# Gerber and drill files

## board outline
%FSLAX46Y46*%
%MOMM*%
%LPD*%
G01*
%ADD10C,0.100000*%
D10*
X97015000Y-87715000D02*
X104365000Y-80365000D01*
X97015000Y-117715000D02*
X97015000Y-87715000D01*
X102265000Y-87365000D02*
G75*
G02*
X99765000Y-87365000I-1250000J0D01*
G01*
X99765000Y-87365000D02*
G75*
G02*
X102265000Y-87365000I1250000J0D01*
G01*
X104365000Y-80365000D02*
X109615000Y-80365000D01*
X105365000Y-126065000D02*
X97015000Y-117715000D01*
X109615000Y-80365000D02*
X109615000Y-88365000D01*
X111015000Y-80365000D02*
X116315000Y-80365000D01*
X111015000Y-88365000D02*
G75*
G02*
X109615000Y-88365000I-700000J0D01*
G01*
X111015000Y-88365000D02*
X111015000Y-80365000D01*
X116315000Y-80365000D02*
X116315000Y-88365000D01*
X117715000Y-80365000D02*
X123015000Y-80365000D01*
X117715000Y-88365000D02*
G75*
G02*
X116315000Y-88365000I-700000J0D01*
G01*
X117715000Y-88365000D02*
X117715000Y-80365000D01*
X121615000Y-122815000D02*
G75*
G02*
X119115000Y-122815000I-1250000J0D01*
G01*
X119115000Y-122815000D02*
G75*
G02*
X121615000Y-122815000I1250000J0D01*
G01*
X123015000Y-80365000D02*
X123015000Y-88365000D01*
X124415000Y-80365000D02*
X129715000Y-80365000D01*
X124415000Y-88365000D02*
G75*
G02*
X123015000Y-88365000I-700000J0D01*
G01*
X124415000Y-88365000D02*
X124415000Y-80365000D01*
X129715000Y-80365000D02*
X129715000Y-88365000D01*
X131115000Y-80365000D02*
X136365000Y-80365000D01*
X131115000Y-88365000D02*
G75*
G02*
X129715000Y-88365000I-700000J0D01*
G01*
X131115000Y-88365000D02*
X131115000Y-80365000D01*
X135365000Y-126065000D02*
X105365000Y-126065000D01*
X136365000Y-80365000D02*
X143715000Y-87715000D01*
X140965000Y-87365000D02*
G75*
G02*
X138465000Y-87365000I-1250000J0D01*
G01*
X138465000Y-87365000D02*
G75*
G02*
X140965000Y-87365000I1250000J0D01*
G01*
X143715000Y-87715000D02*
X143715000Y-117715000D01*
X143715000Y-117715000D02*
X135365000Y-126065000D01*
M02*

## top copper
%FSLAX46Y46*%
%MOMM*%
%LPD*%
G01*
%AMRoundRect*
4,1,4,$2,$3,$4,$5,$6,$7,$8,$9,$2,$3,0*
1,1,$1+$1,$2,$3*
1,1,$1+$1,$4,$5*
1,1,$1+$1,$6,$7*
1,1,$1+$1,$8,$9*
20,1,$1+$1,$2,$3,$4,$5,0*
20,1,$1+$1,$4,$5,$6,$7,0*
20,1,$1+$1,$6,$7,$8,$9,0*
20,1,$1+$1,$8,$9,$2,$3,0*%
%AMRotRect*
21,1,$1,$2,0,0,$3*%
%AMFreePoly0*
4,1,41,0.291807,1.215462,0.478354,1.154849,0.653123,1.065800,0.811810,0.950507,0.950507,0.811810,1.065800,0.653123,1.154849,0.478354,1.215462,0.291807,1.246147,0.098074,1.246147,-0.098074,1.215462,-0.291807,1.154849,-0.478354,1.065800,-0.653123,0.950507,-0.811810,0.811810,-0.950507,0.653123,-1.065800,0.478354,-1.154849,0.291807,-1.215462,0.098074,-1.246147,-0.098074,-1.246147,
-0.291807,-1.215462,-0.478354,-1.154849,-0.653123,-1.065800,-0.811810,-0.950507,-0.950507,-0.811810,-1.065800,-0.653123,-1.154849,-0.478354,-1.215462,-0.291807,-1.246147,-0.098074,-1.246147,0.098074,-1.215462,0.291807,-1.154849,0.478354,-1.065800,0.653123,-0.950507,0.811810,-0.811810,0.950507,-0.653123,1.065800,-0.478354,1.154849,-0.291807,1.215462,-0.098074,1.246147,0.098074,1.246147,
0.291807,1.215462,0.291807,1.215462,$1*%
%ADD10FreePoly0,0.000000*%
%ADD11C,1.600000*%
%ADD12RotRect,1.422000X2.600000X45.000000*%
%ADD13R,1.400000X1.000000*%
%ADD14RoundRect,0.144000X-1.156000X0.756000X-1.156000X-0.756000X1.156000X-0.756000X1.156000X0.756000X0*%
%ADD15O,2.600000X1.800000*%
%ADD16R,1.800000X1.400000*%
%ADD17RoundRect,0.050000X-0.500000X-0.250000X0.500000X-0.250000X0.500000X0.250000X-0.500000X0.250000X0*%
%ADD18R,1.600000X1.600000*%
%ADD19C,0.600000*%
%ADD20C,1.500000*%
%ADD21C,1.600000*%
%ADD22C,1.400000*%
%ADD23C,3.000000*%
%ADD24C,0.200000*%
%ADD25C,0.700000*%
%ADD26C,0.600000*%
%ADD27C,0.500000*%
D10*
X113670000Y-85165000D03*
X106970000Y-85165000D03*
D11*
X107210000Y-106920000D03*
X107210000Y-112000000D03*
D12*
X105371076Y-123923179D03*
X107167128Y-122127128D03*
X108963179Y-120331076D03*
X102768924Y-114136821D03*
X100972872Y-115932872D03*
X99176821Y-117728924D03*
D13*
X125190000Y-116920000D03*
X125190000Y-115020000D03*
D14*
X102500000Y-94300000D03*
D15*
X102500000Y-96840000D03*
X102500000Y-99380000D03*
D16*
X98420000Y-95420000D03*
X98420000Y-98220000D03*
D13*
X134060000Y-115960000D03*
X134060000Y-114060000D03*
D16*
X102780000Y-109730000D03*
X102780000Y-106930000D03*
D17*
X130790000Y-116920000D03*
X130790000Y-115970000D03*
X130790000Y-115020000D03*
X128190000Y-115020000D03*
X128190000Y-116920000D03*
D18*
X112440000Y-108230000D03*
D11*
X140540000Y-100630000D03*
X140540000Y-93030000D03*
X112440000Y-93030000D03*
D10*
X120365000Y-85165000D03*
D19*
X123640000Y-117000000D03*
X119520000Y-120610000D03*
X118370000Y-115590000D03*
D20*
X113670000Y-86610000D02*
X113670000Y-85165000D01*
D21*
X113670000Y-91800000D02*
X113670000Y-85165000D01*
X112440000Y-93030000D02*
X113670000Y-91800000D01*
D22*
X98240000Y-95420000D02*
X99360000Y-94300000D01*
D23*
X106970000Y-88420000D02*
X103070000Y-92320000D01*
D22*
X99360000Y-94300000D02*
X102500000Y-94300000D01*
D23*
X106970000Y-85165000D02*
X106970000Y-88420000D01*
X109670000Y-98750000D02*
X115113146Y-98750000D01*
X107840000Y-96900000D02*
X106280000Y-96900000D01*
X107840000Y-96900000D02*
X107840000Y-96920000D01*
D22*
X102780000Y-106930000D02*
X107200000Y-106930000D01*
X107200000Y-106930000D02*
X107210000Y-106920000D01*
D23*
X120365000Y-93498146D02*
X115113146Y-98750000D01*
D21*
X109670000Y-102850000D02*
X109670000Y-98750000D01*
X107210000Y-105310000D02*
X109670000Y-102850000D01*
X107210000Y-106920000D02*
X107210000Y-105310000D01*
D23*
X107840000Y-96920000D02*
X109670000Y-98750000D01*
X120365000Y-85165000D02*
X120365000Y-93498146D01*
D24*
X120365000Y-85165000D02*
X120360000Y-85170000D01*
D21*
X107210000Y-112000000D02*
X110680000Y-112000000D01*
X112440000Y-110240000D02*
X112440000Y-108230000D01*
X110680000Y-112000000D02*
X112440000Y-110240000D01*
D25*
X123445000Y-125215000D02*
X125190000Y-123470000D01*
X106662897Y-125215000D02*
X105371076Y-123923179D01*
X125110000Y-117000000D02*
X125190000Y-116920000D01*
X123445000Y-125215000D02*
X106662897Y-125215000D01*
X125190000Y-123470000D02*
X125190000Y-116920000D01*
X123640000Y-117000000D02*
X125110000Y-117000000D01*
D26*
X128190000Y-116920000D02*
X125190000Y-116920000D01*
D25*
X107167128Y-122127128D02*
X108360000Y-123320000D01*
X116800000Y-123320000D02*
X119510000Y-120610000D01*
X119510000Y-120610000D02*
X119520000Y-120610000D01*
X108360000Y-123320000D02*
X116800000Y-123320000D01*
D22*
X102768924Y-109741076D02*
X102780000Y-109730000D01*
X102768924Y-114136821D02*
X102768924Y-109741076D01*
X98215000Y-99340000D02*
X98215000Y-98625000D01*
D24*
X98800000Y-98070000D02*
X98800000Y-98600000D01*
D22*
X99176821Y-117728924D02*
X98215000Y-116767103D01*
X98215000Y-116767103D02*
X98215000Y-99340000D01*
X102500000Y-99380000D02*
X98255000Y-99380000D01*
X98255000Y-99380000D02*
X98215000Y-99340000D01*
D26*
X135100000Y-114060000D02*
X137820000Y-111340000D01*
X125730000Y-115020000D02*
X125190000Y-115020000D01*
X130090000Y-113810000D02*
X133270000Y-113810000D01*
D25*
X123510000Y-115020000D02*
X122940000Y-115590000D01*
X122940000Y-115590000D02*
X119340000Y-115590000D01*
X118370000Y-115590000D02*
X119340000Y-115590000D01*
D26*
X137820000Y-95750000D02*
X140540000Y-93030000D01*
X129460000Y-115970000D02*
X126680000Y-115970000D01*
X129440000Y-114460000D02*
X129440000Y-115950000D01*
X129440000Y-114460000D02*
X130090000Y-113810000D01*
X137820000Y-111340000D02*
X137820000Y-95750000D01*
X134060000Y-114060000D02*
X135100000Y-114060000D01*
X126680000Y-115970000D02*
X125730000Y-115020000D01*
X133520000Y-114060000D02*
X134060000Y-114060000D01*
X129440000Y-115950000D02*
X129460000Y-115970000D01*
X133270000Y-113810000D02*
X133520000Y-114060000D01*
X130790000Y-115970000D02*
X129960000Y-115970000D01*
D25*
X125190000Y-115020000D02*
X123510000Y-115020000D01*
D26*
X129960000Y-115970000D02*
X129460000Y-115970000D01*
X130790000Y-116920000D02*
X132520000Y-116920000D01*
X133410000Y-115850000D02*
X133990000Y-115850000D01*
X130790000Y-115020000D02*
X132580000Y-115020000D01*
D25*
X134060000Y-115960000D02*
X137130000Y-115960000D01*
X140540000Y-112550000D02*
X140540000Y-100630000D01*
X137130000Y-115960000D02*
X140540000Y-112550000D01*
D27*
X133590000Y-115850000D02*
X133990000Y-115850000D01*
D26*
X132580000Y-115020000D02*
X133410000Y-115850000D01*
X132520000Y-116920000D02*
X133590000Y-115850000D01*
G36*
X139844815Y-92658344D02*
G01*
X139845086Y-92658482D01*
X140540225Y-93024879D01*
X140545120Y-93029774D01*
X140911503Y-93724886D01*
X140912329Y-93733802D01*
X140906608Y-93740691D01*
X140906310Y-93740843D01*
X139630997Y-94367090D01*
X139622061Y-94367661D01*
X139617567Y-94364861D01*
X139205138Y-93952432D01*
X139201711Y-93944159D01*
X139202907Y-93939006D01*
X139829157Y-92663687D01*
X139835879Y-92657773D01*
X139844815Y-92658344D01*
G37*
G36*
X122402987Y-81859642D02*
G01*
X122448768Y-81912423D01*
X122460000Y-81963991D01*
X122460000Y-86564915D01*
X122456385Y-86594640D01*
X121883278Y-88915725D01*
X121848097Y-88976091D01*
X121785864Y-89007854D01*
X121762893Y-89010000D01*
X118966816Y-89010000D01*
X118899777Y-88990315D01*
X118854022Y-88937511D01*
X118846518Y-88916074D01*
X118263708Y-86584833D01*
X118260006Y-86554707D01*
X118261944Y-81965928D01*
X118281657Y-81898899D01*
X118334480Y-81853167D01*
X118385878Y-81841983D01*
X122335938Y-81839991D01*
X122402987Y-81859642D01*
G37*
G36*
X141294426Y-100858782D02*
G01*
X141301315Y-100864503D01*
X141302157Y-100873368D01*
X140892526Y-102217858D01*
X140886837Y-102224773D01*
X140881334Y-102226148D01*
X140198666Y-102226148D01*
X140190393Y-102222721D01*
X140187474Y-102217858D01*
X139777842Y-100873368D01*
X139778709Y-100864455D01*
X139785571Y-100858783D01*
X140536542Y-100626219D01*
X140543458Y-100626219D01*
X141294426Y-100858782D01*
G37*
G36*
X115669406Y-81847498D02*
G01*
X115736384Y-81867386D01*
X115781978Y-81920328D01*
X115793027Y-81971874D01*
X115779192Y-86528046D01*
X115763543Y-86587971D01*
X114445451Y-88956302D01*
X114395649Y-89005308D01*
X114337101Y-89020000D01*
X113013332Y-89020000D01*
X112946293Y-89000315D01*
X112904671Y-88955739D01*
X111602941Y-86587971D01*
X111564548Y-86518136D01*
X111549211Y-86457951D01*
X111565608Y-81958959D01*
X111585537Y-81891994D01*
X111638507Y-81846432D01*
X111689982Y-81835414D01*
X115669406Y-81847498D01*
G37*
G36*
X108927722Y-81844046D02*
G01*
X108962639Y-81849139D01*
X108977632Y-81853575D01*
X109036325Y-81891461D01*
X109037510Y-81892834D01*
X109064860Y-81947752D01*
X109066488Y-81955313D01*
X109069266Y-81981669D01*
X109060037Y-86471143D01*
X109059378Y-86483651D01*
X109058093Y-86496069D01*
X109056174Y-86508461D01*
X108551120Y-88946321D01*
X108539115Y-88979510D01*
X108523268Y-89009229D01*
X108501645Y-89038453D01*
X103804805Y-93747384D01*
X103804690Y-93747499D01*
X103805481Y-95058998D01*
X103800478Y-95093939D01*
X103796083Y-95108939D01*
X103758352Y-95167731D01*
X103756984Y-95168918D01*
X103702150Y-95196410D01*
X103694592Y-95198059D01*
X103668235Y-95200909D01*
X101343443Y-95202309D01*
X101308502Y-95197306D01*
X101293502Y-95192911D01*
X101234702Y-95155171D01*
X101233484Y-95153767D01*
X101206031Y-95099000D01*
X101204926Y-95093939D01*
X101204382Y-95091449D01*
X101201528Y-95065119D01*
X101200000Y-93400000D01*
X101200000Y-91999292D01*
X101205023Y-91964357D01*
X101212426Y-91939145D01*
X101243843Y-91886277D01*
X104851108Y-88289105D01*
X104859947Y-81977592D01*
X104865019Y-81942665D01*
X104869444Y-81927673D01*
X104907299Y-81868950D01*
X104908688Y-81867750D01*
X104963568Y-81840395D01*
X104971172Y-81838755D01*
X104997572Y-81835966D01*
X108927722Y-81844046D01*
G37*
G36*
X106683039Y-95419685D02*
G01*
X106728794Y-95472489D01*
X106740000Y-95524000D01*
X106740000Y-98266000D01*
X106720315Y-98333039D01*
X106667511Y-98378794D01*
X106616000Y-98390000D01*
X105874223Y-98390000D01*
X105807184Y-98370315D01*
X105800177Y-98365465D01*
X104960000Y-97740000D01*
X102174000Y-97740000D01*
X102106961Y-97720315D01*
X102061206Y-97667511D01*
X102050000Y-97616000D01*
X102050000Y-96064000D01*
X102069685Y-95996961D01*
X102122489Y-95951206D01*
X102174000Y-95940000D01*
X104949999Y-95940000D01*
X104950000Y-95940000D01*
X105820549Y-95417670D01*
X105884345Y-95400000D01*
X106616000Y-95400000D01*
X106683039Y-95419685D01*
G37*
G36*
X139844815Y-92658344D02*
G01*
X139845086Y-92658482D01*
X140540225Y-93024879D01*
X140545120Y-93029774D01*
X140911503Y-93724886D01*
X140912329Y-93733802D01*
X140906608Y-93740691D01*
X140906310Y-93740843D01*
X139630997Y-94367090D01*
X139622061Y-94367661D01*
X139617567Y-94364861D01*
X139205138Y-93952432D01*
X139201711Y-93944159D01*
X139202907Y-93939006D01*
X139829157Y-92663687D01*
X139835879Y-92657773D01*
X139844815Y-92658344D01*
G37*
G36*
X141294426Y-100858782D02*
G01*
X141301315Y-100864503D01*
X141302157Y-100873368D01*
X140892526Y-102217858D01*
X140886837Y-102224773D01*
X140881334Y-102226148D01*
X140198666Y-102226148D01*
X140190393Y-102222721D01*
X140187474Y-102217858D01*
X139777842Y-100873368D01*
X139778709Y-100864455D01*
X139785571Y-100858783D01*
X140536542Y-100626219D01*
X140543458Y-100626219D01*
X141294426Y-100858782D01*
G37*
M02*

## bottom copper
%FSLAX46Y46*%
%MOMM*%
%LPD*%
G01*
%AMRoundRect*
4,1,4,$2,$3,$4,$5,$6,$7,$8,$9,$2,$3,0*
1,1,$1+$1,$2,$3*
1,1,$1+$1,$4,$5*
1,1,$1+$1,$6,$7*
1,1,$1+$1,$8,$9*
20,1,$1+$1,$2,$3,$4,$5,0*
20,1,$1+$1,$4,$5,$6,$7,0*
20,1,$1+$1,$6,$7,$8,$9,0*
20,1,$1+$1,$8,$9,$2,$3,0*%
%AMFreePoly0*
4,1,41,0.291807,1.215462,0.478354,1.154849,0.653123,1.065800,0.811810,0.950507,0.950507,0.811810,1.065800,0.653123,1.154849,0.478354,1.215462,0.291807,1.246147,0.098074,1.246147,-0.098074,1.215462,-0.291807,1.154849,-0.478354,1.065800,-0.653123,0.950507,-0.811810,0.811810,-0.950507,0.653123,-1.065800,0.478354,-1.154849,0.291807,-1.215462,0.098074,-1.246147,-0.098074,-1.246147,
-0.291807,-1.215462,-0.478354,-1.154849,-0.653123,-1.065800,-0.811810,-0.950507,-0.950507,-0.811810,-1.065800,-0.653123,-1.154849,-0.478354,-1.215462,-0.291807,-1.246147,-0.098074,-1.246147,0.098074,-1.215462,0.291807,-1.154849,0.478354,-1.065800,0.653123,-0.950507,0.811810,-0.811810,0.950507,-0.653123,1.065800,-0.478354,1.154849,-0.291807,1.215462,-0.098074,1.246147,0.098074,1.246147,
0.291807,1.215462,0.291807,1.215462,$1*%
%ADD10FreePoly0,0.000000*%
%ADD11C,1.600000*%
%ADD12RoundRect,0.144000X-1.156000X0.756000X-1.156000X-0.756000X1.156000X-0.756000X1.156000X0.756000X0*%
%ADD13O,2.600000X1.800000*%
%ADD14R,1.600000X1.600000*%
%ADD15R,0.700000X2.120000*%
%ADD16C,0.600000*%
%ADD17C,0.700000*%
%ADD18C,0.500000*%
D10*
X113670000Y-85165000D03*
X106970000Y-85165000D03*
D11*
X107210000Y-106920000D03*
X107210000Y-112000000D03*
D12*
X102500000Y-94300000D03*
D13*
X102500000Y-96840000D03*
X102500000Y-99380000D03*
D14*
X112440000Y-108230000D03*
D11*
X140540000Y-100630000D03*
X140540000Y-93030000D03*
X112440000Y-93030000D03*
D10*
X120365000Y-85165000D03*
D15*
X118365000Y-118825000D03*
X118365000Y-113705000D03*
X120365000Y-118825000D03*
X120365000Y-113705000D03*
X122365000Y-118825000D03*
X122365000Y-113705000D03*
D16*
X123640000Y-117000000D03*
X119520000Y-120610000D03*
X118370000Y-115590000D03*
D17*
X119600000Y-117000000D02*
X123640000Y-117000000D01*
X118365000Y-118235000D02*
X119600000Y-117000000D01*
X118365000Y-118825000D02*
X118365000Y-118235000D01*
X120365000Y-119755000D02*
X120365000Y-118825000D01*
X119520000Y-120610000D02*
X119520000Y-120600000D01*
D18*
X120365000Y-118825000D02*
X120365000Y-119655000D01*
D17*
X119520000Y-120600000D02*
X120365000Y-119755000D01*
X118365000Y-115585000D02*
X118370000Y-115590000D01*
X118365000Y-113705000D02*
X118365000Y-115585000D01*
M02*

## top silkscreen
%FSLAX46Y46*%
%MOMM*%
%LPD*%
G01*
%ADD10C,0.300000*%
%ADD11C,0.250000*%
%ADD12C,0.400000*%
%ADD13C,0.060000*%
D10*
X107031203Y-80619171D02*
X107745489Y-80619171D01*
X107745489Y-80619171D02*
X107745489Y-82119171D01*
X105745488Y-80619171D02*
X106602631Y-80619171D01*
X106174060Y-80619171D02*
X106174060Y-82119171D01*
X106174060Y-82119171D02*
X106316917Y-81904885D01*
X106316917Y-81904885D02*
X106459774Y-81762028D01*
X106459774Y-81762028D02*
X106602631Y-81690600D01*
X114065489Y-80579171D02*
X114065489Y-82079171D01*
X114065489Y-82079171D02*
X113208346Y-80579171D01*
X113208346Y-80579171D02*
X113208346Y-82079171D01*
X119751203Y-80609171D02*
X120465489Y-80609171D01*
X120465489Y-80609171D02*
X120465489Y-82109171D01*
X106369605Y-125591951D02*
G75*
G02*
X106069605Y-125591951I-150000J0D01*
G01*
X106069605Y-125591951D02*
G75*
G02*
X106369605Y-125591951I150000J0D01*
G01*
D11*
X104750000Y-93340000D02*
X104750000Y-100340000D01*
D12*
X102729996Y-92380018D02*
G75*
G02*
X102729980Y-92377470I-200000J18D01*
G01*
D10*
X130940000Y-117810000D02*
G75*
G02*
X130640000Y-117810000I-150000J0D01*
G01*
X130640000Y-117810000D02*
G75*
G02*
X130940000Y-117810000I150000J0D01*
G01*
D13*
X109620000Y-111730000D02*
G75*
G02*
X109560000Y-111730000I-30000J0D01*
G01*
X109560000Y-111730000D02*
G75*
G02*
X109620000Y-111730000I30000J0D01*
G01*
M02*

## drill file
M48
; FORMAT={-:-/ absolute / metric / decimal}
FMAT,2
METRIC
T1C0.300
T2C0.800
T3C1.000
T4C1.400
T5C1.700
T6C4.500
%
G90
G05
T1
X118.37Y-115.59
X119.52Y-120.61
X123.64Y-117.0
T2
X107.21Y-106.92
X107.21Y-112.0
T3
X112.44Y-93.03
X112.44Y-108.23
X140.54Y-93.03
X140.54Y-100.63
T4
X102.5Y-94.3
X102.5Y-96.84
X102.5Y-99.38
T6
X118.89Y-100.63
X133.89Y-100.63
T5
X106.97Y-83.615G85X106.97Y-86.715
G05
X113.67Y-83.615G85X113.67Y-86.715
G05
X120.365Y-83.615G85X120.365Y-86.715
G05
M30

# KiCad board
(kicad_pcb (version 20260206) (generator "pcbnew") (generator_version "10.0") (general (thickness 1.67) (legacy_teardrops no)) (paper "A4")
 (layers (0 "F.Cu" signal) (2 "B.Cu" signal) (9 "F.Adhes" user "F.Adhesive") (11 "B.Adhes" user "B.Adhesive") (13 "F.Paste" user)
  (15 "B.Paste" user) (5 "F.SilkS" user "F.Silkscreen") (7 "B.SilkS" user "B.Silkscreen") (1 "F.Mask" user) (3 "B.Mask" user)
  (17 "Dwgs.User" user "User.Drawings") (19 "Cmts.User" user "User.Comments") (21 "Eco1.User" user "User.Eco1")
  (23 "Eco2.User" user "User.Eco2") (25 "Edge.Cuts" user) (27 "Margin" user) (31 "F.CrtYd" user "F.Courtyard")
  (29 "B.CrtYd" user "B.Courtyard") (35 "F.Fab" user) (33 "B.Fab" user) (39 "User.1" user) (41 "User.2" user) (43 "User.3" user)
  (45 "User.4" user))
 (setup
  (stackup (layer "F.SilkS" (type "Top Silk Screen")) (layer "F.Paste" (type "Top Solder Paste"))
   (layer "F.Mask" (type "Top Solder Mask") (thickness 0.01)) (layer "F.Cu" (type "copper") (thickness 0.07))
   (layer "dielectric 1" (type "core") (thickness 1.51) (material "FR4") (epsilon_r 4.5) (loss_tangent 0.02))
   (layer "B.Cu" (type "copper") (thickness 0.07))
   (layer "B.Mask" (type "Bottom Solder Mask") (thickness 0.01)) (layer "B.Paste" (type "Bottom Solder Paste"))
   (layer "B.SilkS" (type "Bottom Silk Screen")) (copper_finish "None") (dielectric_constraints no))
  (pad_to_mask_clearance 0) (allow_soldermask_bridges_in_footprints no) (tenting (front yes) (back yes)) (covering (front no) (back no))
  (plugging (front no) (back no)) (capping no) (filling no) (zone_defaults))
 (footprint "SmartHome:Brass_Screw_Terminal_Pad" (layer "F.Cu") (at 113.67 85.165)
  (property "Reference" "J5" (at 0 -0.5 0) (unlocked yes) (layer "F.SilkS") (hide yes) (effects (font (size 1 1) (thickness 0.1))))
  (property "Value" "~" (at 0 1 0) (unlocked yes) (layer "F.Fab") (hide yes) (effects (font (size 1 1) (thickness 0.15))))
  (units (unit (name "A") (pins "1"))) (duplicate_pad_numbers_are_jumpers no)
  (pad "1" thru_hole custom (at 0 0) (size 2.5 2.5) (drill oval 1.7 4.8) (layers "*.Cu" "*.Mask") (remove_unused_layers no) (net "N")
   (options (clearance outline) (anchor circle)) (primitives)))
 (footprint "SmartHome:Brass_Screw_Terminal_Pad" (layer "F.Cu") (at 106.97 85.165)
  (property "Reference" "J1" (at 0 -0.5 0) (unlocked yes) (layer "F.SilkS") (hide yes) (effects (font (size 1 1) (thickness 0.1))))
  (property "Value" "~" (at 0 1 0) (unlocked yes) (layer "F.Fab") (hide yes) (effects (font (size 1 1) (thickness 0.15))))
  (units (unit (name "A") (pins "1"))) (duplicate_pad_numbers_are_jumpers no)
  (pad "1" thru_hole custom (at 0 0) (size 2.5 2.5) (drill oval 1.7 4.8) (layers "*.Cu" "*.Mask") (remove_unused_layers no) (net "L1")
   (options (clearance outline) (anchor circle)) (primitives)))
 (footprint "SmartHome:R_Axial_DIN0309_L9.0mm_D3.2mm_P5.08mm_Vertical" (layer "F.Cu") (at 107.21 106.92 -90)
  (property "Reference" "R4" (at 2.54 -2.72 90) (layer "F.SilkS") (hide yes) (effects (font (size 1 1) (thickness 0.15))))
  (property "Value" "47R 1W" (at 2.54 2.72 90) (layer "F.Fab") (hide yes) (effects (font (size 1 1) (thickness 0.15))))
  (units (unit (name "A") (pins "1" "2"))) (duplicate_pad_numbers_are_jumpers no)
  (pad "1" thru_hole circle (at 0 0 270) (size 1.6 1.6) (drill 0.8) (layers "*.Cu" "*.Mask") (remove_unused_layers no) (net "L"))
  (pad "2" thru_hole circle (at 5.08 0 270) (size 1.6 1.6) (drill 0.8) (layers "*.Cu" "*.Mask") (remove_unused_layers no)
   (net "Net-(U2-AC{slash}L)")))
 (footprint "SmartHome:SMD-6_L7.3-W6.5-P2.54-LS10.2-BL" (layer "F.Cu") (at 104.07 119.03 45)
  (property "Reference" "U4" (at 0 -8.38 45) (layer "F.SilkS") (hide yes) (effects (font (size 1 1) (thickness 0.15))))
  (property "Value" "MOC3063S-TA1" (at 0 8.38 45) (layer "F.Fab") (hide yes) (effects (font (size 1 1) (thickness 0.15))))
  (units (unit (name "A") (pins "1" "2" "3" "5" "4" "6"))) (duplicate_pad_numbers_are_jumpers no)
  (fp_circle (center -3.12 6.16) (end -2.97 6.16) (stroke (width 0.3) (type solid)) (fill no) (layer "F.SilkS"))
  (pad "1" smd rect (at -2.54 4.38 45) (size 1.422 2.6) (layers "F.Cu" "F.Mask" "F.Paste") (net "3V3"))
  (pad "2" smd rect (at 0 4.38 45) (size 1.422 2.6) (layers "F.Cu" "F.Mask" "F.Paste") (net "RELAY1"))
  (pad "3" smd rect (at 2.54 4.38 45) (size 1.422 2.6) (layers "F.Cu" "F.Mask" "F.Paste") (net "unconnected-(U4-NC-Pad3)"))
  (pad "4" smd rect (at 2.54 -4.38 45) (size 1.422 2.6) (layers "F.Cu" "F.Mask" "F.Paste") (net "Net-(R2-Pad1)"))
  (pad "5" smd rect (at 0 -4.38 45) (size 1.422 2.6) (layers "F.Cu" "F.Mask" "F.Paste") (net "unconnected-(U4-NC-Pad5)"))
  (pad "6" smd rect (at -2.54 -4.38 45) (size 1.422 2.6) (layers "F.Cu" "F.Mask" "F.Paste") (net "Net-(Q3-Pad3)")))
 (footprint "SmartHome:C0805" (layer "F.Cu") (at 125.19 115.97 90)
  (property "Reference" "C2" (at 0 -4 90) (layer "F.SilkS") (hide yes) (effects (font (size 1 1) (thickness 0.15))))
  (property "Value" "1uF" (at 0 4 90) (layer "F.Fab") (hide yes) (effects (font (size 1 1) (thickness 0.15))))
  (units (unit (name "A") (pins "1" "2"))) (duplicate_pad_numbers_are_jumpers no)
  (pad "1" smd rect (at -0.95 0 90) (size 1 1.4) (layers "F.Cu" "F.Mask" "F.Paste") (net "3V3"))
  (pad "2" smd rect (at 0.95 0 90) (size 1 1.4) (layers "F.Cu" "F.Mask" "F.Paste") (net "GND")))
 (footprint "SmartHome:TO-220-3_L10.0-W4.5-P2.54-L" (layer "F.Cu") (at 102.5 96.84 -90)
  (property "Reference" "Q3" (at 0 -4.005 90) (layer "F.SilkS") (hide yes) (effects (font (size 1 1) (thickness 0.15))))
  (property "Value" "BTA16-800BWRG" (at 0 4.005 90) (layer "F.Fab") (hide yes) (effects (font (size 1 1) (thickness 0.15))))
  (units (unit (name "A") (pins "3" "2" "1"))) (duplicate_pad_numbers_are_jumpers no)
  (fp_line (start -3.5 -2.25) (end 3.5 -2.25) (stroke (width 0.25) (type solid)) (layer "F.SilkS"))
  (fp_arc (start -4.459982 -0.229996) (mid -4.458708 0.17) (end -4.46253 -0.22998) (stroke (width 0.4) (type solid)) (layer "F.SilkS"))
  (pad "1" thru_hole roundrect (at -2.54 0 270) (size 1.8 2.6) (drill 1.4) (layers "*.Cu" "*.Mask") (remove_unused_layers no)
   (roundrect_rratio 0.08) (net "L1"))
  (pad "2" thru_hole oval (at 0 0 270) (size 1.8 2.6) (drill 1.4) (layers "*.Cu" "*.Mask") (remove_unused_layers no) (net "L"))
  (pad "3" thru_hole oval (at 2.54 0 270) (size 1.8 2.6) (drill 1.4) (layers "*.Cu" "*.Mask") (remove_unused_layers no)
   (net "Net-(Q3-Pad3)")))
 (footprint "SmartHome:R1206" (layer "F.Cu") (at 98.42 96.82 -90)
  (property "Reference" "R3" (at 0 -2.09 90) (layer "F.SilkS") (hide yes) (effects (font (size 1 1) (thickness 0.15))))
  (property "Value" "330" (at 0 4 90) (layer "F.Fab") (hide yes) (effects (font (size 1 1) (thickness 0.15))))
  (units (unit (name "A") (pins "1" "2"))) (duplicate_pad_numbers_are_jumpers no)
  (pad "1" smd rect (at -1.4 0 270) (size 1.4 1.8) (layers "F.Cu" "F.Mask" "F.Paste") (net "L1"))
  (pad "2" smd rect (at 1.4 0 270) (size 1.4 1.8) (layers "F.Cu" "F.Mask" "F.Paste") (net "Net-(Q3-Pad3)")))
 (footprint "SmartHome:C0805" (layer "F.Cu") (at 134.06 115.01 90)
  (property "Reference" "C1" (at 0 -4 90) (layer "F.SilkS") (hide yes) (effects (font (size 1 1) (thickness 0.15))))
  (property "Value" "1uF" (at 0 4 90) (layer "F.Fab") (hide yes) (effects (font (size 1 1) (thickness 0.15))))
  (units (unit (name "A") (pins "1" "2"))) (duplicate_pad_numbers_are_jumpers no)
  (pad "1" smd rect (at -0.95 0 90) (size 1 1.4) (layers "F.Cu" "F.Mask" "F.Paste") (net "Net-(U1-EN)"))
  (pad "2" smd rect (at 0.95 0 90) (size 1 1.4) (layers "F.Cu" "F.Mask" "F.Paste") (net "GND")))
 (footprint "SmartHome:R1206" (layer "F.Cu") (at 102.78 108.33 90)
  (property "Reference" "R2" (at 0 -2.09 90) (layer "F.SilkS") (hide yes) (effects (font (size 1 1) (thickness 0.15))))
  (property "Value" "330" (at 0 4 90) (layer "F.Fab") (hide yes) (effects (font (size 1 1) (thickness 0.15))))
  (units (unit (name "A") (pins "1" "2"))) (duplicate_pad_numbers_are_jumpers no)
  (pad "1" smd rect (at -1.4 0 90) (size 1.4 1.8) (layers "F.Cu" "F.Mask" "F.Paste") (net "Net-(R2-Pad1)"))
  (pad "2" smd rect (at 1.4 0 90) (size 1.4 1.8) (layers "F.Cu" "F.Mask" "F.Paste") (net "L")))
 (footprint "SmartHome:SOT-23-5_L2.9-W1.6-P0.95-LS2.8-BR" (layer "F.Cu") (at 129.49 115.97)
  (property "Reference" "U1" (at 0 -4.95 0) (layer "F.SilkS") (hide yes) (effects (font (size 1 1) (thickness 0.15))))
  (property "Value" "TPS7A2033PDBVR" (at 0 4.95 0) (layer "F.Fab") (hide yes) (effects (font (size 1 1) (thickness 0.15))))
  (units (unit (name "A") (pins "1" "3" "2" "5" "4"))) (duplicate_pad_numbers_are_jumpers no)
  (fp_circle (center 1.3 1.84) (end 1.45 1.84) (stroke (width 0.3) (type solid)) (fill no) (layer "F.SilkS"))
  (pad "1" smd roundrect (at 1.3 0.95) (size 1.1 0.6) (layers "F.Cu" "F.Mask" "F.Paste") (roundrect_rratio 0.08333333333)
   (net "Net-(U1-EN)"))
  (pad "2" smd roundrect (at 1.3 0) (size 1.1 0.6) (layers "F.Cu" "F.Mask" "F.Paste") (roundrect_rratio 0.08333333333) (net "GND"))
  (pad "3" smd roundrect (at 1.3 -0.95) (size 1.1 0.6) (layers "F.Cu" "F.Mask" "F.Paste") (roundrect_rratio 0.08333333333)
   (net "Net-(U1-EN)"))
  (pad "4" smd roundrect (at -1.3 -0.95) (size 1.1 0.6) (layers "F.Cu" "F.Mask" "F.Paste") (roundrect_rratio 0.08333333333)
   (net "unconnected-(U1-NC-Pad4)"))
  (pad "5" smd roundrect (at -1.3 0.95) (size 1.1 0.6) (layers "F.Cu" "F.Mask" "F.Paste") (roundrect_rratio 0.08333333333) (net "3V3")))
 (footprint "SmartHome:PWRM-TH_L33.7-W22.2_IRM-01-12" (layer "F.Cu") (at 126.49 100.63)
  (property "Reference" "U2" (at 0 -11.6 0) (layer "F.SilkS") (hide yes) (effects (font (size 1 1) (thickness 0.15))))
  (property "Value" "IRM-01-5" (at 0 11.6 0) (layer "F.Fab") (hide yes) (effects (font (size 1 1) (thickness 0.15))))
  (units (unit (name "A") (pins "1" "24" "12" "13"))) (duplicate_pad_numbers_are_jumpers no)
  (fp_circle (center -16.9 11.1) (end -16.87 11.1) (stroke (width 0.06) (type solid)) (fill no) (layer "F.SilkS"))
  (pad "" np_thru_hole circle (at -7.6 0) (size 4.5 4.5) (drill 4.5) (layers "*.Cu" "*.Mask"))
  (pad "" np_thru_hole circle (at 7.4 0) (size 4.5 4.5) (drill 4.5) (layers "*.Cu" "*.Mask"))
  (pad "1" thru_hole rect (at -14.05 7.6) (size 1.6 1.6) (drill 0.999998) (layers "*.Cu" "*.Mask") (remove_unused_layers no)
   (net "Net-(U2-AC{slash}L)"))
  (pad "12" thru_hole circle (at 14.05 0) (size 1.6 1.6) (drill 0.999998) (layers "*.Cu" "*.Mask") (remove_unused_layers no)
   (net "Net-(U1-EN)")
   (teardrops (best_length_ratio 0.5) (max_length 1) (best_width_ratio 1) (max_width 2) (curved_edges no) (filter_ratio 0.9) (enabled yes)
    (allow_two_segments yes) (prefer_zone_connections yes)))
  (pad "13" thru_hole circle (at 14.05 -7.6) (size 1.6 1.6) (drill 0.999998) (layers "*.Cu" "*.Mask") (remove_unused_layers no) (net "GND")
   (teardrops (best_length_ratio 0.5) (max_length 1) (best_width_ratio 1) (max_width 2) (curved_edges no) (filter_ratio 0.9) (enabled yes)
    (allow_two_segments yes) (prefer_zone_connections yes)))
  (pad "24" thru_hole circle (at -14.05 -7.6) (size 1.6 1.6) (drill 0.999998) (layers "*.Cu" "*.Mask") (remove_unused_layers no) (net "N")))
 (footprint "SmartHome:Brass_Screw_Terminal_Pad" (layer "F.Cu") (at 120.365 85.165)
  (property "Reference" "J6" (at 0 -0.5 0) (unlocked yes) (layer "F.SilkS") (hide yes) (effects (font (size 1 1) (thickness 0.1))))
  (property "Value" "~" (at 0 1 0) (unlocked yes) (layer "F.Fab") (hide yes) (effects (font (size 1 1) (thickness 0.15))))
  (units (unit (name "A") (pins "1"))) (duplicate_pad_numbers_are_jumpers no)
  (pad "1" thru_hole custom (at 0 0) (size 2.5 2.5) (drill oval 1.7 4.8) (layers "*.Cu" "*.Mask") (remove_unused_layers no) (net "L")
   (options (clearance outline) (anchor circle)) (primitives)))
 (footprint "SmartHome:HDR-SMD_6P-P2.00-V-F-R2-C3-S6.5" (layer "B.Cu") (at 120.365 116.265)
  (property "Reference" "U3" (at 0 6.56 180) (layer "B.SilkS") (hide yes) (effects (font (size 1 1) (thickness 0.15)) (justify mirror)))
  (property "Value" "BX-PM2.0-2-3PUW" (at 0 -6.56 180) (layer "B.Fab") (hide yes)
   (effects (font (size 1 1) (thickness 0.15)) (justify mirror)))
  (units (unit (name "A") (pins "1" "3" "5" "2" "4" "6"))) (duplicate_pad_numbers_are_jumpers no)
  (pad "1" smd rect (at -2 2.56) (size 0.7 2.12) (layers "B.Cu" "B.Mask" "B.Paste") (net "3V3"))
  (pad "2" smd rect (at -2 -2.56) (size 0.7 2.12) (layers "B.Cu" "B.Mask" "B.Paste") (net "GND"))
  (pad "3" smd rect (at 0 2.56) (size 0.7 2.12) (layers "B.Cu" "B.Mask" "B.Paste") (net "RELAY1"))
  (pad "4" smd rect (at 0 -2.56) (size 0.7 2.12) (layers "B.Cu" "B.Mask" "B.Paste") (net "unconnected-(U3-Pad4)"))
  (pad "5" smd rect (at 2 2.56) (size 0.7 2.12) (layers "B.Cu" "B.Mask" "B.Paste") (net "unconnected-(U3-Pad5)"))
  (pad "6" smd rect (at 2 -2.56) (size 0.7 2.12) (layers "B.Cu" "B.Mask" "B.Paste") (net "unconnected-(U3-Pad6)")))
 (gr_line (start 97.015 87.715) (end 104.365 80.365) (stroke (width 0.1) (type default)) (layer "Edge.Cuts"))
 (gr_line (start 97.015 117.715) (end 97.015 87.715) (stroke (width 0.1) (type default)) (layer "Edge.Cuts"))
 (gr_circle (center 101.015 87.365) (end 102.265 87.365) (stroke (width 0.1) (type default)) (fill no) (layer "Edge.Cuts"))
 (gr_line (start 104.365 80.365) (end 109.615 80.365) (stroke (width 0.1) (type default)) (layer "Edge.Cuts"))
 (gr_line (start 105.365 126.065) (end 97.015 117.715) (stroke (width 0.1) (type default)) (layer "Edge.Cuts"))
 (gr_line (start 109.615 80.365) (end 109.615 88.365) (stroke (width 0.1) (type default)) (layer "Edge.Cuts"))
 (gr_line (start 111.015 80.365) (end 116.315 80.365) (stroke (width 0.1) (type default)) (layer "Edge.Cuts"))
 (gr_arc (start 111.015 88.365) (mid 110.315 89.065) (end 109.615 88.365) (stroke (width 0.1) (type default)) (layer "Edge.Cuts"))
 (gr_line (start 111.015 88.365) (end 111.015 80.365) (stroke (width 0.1) (type default)) (layer "Edge.Cuts"))
 (gr_line (start 116.315 80.365) (end 116.315 88.365) (stroke (width 0.1) (type default)) (layer "Edge.Cuts"))
 (gr_line (start 117.715 80.365) (end 123.015 80.365) (stroke (width 0.1) (type default)) (layer "Edge.Cuts"))
 (gr_arc (start 117.715 88.365) (mid 117.015 89.065) (end 116.315 88.365) (stroke (width 0.1) (type default)) (layer "Edge.Cuts"))
 (gr_line (start 117.715 88.365) (end 117.715 80.365) (stroke (width 0.1) (type default)) (layer "Edge.Cuts"))
 (gr_circle (center 120.365 122.815) (end 121.615 122.815) (stroke (width 0.1) (type default)) (fill no) (layer "Edge.Cuts"))
 (gr_line (start 123.015 80.365) (end 123.015 88.365) (stroke (width 0.1) (type default)) (layer "Edge.Cuts"))
 (gr_line (start 124.415 80.365) (end 129.715 80.365) (stroke (width 0.1) (type default)) (layer "Edge.Cuts"))
 (gr_arc (start 124.415 88.365) (mid 123.715 89.065) (end 123.015 88.365) (stroke (width 0.1) (type default)) (layer "Edge.Cuts"))
 (gr_line (start 124.415 88.365) (end 124.415 80.365) (stroke (width 0.1) (type default)) (layer "Edge.Cuts"))
 (gr_line (start 129.715 80.365) (end 129.715 88.365) (stroke (width 0.1) (type default)) (layer "Edge.Cuts"))
 (gr_line (start 131.115 80.365) (end 136.365 80.365) (stroke (width 0.1) (type default)) (layer "Edge.Cuts"))
 (gr_arc (start 131.115 88.365) (mid 130.415 89.065) (end 129.715 88.365) (stroke (width 0.1) (type default)) (layer "Edge.Cuts"))
 (gr_line (start 131.115 88.365) (end 131.115 80.365) (stroke (width 0.1) (type default)) (layer "Edge.Cuts"))
 (gr_line (start 135.365 126.065) (end 105.365 126.065) (stroke (width 0.1) (type default)) (layer "Edge.Cuts"))
 (gr_line (start 136.365 80.365) (end 143.715 87.715) (stroke (width 0.1) (type default)) (layer "Edge.Cuts"))
 (gr_circle (center 139.715 87.365) (end 140.965 87.365) (stroke (width 0.1) (type default)) (fill no) (layer "Edge.Cuts"))
 (gr_line (start 143.715 87.715) (end 143.715 117.715) (stroke (width 0.1) (type default)) (layer "Edge.Cuts"))
 (gr_line (start 143.715 117.715) (end 135.365 126.065) (stroke (width 0.1) (type default)) (layer "Edge.Cuts"))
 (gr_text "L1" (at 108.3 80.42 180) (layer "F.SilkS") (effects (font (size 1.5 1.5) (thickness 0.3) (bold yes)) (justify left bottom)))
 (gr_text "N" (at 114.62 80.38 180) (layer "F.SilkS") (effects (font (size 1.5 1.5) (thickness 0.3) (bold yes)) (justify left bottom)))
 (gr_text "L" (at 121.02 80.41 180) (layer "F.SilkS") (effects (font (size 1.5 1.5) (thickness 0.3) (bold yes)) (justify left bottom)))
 (segment (start 113.67 86.61) (end 113.67 85.165) (width 1.5) (layer "F.Cu") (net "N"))
 (segment (start 113.67 91.8) (end 113.67 85.165) (width 1.6) (layer "F.Cu") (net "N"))
 (segment (start 112.44 93.03) (end 113.67 91.8) (width 1.6) (layer "F.Cu") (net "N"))
 (segment (start 98.24 95.42) (end 99.36 94.3) (width 1.4) (layer "F.Cu") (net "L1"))
 (segment (start 106.97 88.42) (end 103.07 92.32) (width 3) (layer "F.Cu") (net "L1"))
 (segment (start 99.36 94.3) (end 102.5 94.3) (width 1.4) (layer "F.Cu") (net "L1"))
 (segment (start 106.97 85.165) (end 106.97 88.42) (width 3) (layer "F.Cu") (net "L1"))
 (segment (start 109.67 98.75) (end 115.113146 98.75) (width 3) (layer "F.Cu") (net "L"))
 (segment (start 107.84 96.9) (end 106.28 96.9) (width 3) (layer "F.Cu") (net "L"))
 (segment (start 107.84 96.9) (end 107.84 96.92) (width 3) (layer "F.Cu") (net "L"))
 (segment (start 102.78 106.93) (end 107.2 106.93) (width 1.4) (layer "F.Cu") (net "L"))
 (segment (start 107.2 106.93) (end 107.21 106.92) (width 1.4) (layer "F.Cu") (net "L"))
 (segment (start 120.365 93.498146) (end 115.113146 98.75) (width 3) (layer "F.Cu") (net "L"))
 (segment (start 109.67 102.85) (end 109.67 98.75) (width 1.6) (layer "F.Cu") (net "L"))
 (segment (start 107.21 105.31) (end 109.67 102.85) (width 1.6) (layer "F.Cu") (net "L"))
 (segment (start 107.21 106.92) (end 107.21 105.31) (width 1.6) (layer "F.Cu") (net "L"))
 (segment (start 107.84 96.92) (end 109.67 98.75) (width 3) (layer "F.Cu") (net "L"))
 (segment (start 120.365 85.165) (end 120.365 93.498146) (width 3) (layer "F.Cu") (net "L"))
 (segment (start 120.365 85.165) (end 120.36 85.17) (width 0.2) (layer "F.Cu") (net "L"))
 (segment (start 107.21 112) (end 110.68 112) (width 1.6) (layer "F.Cu") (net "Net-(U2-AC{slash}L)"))
 (segment (start 112.44 110.24) (end 112.44 108.23) (width 1.6) (layer "F.Cu") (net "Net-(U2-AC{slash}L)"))
 (segment (start 110.68 112) (end 112.44 110.24) (width 1.6) (layer "F.Cu") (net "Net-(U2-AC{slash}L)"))
 (segment (start 123.445 125.215) (end 125.19 123.47) (width 0.7) (layer "F.Cu") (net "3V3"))
 (segment (start 106.662897 125.215) (end 105.371076 123.923179) (width 0.7) (layer "F.Cu") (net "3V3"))
 (segment (start 125.11 117) (end 125.19 116.92) (width 0.7) (layer "F.Cu") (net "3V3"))
 (segment (start 123.445 125.215) (end 106.662897 125.215) (width 0.7) (layer "F.Cu") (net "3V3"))
 (segment (start 125.19 123.47) (end 125.19 116.92) (width 0.7) (layer "F.Cu") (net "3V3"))
 (segment (start 123.64 117) (end 125.11 117) (width 0.7) (layer "F.Cu") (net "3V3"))
 (segment (start 128.19 116.92) (end 125.19 116.92) (width 0.6) (layer "F.Cu") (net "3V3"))
 (via (at 123.64 117) (size 0.6) (drill 0.3) (layers "F.Cu" "B.Cu") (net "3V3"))
 (segment (start 119.6 117) (end 123.64 117) (width 0.7) (layer "B.Cu") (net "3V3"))
 (segment (start 118.365 118.235) (end 119.6 117) (width 0.7) (layer "B.Cu") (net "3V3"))
 (segment (start 118.365 118.825) (end 118.365 118.235) (width 0.7) (layer "B.Cu") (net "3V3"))
 (segment (start 107.167128 122.127128) (end 108.36 123.32) (width 0.7) (layer "F.Cu") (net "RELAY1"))
 (segment (start 116.8 123.32) (end 119.51 120.61) (width 0.7) (layer "F.Cu") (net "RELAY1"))
 (segment (start 119.51 120.61) (end 119.52 120.61) (width 0.7) (layer "F.Cu") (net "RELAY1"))
 (segment (start 108.36 123.32) (end 116.8 123.32) (width 0.7) (layer "F.Cu") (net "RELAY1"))
 (via (at 119.52 120.61) (size 0.6) (drill 0.3) (layers "F.Cu" "B.Cu") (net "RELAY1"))
 (segment (start 120.365 119.755) (end 120.365 118.825) (width 0.7) (layer "B.Cu") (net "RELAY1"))
 (segment (start 119.52 120.61) (end 119.52 120.6) (width 0.7) (layer "B.Cu") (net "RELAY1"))
 (segment (start 120.365 118.825) (end 120.365 119.655) (width 0.5) (layer "B.Cu") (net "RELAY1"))
 (segment (start 119.52 120.6) (end 120.365 119.755) (width 0.7) (layer "B.Cu") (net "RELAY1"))
 (segment (start 102.768924 109.741076) (end 102.78 109.73) (width 1.4) (layer "F.Cu") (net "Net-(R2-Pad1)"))
 (segment (start 102.768924 114.136821) (end 102.768924 109.741076) (width 1.4) (layer "F.Cu") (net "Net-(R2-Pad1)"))
 (segment (start 98.215 99.34) (end 98.215 98.625) (width 1.4) (layer "F.Cu") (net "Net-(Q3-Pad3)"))
 (segment (start 98.8 98.07) (end 98.8 98.6) (width 0.2) (layer "F.Cu") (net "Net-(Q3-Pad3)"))
 (segment (start 99.176821 117.728924) (end 98.215 116.767103) (width 1.4) (layer "F.Cu") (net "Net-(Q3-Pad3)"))
 (segment (start 98.215 116.767103) (end 98.215 99.34) (width 1.4) (layer "F.Cu") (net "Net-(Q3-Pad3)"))
 (segment (start 102.5 99.38) (end 98.255 99.38) (width 1.4) (layer "F.Cu") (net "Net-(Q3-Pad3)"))
 (segment (start 98.255 99.38) (end 98.215 99.34) (width 1.4) (layer "F.Cu") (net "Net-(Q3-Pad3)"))
 (segment (start 135.1 114.06) (end 137.82 111.34) (width 0.6) (layer "F.Cu") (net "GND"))
 (segment (start 125.73 115.02) (end 125.19 115.02) (width 0.6) (layer "F.Cu") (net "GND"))
 (segment (start 130.09 113.81) (end 133.27 113.81) (width 0.6) (layer "F.Cu") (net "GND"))
 (segment (start 123.51 115.02) (end 122.94 115.59) (width 0.7) (layer "F.Cu") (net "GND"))
 (segment (start 122.94 115.59) (end 119.34 115.59) (width 0.7) (layer "F.Cu") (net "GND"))
 (segment (start 118.37 115.59) (end 119.34 115.59) (width 0.7) (layer "F.Cu") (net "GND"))
 (segment (start 137.82 95.75) (end 140.54 93.03) (width 0.6) (layer "F.Cu") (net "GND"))
 (segment (start 129.46 115.97) (end 126.68 115.97) (width 0.6) (layer "F.Cu") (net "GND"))
 (segment (start 129.44 114.46) (end 129.44 115.95) (width 0.6) (layer "F.Cu") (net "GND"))
 (segment (start 129.44 114.46) (end 130.09 113.81) (width 0.6) (layer "F.Cu") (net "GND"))
 (segment (start 137.82 111.34) (end 137.82 95.75) (width 0.6) (layer "F.Cu") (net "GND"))
 (segment (start 134.06 114.06) (end 135.1 114.06) (width 0.6) (layer "F.Cu") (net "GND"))
 (segment (start 126.68 115.97) (end 125.73 115.02) (width 0.6) (layer "F.Cu") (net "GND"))
 (segment (start 133.52 114.06) (end 134.06 114.06) (width 0.6) (layer "F.Cu") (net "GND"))
 (segment (start 129.44 115.95) (end 129.46 115.97) (width 0.6) (layer "F.Cu") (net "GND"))
 (segment (start 133.27 113.81) (end 133.52 114.06) (width 0.6) (layer "F.Cu") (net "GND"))
 (segment (start 130.79 115.97) (end 129.96 115.97) (width 0.6) (layer "F.Cu") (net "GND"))
 (segment (start 125.19 115.02) (end 123.51 115.02) (width 0.7) (layer "F.Cu") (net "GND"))
 (segment (start 129.96 115.97) (end 129.46 115.97) (width 0.6) (layer "F.Cu") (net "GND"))
 (via (at 118.37 115.59) (size 0.6) (drill 0.3) (layers "F.Cu" "B.Cu") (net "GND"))
 (segment (start 118.365 115.585) (end 118.37 115.59) (width 0.7) (layer "B.Cu") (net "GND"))
 (segment (start 118.365 113.705) (end 118.365 115.585) (width 0.7) (layer "B.Cu") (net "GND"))
 (segment (start 130.79 116.92) (end 132.52 116.92) (width 0.6) (layer "F.Cu") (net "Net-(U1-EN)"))
 (segment (start 133.41 115.85) (end 133.99 115.85) (width 0.6) (layer "F.Cu") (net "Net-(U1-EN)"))
 (segment (start 130.79 115.02) (end 132.58 115.02) (width 0.6) (layer "F.Cu") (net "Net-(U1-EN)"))
 (segment (start 134.06 115.96) (end 137.13 115.96) (width 0.7) (layer "F.Cu") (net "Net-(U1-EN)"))
 (segment (start 140.54 112.55) (end 140.54 100.63) (width 0.7) (layer "F.Cu") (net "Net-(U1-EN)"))
 (segment (start 137.13 115.96) (end 140.54 112.55) (width 0.7) (layer "F.Cu") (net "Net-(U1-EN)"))
 (segment (start 133.59 115.85) (end 133.99 115.85) (width 0.5) (layer "F.Cu") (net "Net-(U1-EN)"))
 (segment (start 132.58 115.02) (end 133.41 115.85) (width 0.6) (layer "F.Cu") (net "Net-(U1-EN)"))
 (segment (start 132.52 116.92) (end 133.59 115.85) (width 0.6) (layer "F.Cu") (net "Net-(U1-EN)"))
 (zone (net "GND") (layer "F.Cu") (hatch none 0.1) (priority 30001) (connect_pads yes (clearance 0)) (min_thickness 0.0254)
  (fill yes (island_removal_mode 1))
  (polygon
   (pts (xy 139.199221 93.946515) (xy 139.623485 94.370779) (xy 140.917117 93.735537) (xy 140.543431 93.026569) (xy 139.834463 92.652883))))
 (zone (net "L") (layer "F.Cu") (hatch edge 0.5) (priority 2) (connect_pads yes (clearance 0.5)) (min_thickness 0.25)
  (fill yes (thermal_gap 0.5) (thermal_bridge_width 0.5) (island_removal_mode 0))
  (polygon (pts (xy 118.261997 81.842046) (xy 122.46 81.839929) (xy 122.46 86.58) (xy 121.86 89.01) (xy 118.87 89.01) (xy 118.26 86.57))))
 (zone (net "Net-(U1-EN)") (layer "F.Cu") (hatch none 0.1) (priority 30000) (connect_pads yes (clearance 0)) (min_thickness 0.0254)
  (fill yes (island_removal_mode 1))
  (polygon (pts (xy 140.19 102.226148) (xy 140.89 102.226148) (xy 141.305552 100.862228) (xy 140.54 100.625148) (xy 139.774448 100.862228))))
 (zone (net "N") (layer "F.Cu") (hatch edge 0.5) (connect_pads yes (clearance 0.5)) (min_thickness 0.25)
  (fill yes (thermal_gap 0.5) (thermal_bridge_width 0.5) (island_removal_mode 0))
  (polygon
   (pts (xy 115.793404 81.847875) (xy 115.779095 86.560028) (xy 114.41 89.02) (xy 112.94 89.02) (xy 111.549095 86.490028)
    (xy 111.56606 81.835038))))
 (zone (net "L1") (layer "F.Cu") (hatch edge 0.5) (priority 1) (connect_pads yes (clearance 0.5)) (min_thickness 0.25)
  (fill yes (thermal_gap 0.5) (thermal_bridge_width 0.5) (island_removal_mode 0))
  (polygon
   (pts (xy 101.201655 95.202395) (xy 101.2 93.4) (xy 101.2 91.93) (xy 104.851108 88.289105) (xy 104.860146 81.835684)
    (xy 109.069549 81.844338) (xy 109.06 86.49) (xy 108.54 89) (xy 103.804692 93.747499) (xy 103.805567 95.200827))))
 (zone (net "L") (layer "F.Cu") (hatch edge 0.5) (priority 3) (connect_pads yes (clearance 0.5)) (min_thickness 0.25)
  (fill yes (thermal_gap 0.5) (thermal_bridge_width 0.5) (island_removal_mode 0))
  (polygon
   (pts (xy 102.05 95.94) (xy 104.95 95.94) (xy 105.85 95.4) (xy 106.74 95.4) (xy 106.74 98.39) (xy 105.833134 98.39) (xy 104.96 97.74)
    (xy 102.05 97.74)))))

